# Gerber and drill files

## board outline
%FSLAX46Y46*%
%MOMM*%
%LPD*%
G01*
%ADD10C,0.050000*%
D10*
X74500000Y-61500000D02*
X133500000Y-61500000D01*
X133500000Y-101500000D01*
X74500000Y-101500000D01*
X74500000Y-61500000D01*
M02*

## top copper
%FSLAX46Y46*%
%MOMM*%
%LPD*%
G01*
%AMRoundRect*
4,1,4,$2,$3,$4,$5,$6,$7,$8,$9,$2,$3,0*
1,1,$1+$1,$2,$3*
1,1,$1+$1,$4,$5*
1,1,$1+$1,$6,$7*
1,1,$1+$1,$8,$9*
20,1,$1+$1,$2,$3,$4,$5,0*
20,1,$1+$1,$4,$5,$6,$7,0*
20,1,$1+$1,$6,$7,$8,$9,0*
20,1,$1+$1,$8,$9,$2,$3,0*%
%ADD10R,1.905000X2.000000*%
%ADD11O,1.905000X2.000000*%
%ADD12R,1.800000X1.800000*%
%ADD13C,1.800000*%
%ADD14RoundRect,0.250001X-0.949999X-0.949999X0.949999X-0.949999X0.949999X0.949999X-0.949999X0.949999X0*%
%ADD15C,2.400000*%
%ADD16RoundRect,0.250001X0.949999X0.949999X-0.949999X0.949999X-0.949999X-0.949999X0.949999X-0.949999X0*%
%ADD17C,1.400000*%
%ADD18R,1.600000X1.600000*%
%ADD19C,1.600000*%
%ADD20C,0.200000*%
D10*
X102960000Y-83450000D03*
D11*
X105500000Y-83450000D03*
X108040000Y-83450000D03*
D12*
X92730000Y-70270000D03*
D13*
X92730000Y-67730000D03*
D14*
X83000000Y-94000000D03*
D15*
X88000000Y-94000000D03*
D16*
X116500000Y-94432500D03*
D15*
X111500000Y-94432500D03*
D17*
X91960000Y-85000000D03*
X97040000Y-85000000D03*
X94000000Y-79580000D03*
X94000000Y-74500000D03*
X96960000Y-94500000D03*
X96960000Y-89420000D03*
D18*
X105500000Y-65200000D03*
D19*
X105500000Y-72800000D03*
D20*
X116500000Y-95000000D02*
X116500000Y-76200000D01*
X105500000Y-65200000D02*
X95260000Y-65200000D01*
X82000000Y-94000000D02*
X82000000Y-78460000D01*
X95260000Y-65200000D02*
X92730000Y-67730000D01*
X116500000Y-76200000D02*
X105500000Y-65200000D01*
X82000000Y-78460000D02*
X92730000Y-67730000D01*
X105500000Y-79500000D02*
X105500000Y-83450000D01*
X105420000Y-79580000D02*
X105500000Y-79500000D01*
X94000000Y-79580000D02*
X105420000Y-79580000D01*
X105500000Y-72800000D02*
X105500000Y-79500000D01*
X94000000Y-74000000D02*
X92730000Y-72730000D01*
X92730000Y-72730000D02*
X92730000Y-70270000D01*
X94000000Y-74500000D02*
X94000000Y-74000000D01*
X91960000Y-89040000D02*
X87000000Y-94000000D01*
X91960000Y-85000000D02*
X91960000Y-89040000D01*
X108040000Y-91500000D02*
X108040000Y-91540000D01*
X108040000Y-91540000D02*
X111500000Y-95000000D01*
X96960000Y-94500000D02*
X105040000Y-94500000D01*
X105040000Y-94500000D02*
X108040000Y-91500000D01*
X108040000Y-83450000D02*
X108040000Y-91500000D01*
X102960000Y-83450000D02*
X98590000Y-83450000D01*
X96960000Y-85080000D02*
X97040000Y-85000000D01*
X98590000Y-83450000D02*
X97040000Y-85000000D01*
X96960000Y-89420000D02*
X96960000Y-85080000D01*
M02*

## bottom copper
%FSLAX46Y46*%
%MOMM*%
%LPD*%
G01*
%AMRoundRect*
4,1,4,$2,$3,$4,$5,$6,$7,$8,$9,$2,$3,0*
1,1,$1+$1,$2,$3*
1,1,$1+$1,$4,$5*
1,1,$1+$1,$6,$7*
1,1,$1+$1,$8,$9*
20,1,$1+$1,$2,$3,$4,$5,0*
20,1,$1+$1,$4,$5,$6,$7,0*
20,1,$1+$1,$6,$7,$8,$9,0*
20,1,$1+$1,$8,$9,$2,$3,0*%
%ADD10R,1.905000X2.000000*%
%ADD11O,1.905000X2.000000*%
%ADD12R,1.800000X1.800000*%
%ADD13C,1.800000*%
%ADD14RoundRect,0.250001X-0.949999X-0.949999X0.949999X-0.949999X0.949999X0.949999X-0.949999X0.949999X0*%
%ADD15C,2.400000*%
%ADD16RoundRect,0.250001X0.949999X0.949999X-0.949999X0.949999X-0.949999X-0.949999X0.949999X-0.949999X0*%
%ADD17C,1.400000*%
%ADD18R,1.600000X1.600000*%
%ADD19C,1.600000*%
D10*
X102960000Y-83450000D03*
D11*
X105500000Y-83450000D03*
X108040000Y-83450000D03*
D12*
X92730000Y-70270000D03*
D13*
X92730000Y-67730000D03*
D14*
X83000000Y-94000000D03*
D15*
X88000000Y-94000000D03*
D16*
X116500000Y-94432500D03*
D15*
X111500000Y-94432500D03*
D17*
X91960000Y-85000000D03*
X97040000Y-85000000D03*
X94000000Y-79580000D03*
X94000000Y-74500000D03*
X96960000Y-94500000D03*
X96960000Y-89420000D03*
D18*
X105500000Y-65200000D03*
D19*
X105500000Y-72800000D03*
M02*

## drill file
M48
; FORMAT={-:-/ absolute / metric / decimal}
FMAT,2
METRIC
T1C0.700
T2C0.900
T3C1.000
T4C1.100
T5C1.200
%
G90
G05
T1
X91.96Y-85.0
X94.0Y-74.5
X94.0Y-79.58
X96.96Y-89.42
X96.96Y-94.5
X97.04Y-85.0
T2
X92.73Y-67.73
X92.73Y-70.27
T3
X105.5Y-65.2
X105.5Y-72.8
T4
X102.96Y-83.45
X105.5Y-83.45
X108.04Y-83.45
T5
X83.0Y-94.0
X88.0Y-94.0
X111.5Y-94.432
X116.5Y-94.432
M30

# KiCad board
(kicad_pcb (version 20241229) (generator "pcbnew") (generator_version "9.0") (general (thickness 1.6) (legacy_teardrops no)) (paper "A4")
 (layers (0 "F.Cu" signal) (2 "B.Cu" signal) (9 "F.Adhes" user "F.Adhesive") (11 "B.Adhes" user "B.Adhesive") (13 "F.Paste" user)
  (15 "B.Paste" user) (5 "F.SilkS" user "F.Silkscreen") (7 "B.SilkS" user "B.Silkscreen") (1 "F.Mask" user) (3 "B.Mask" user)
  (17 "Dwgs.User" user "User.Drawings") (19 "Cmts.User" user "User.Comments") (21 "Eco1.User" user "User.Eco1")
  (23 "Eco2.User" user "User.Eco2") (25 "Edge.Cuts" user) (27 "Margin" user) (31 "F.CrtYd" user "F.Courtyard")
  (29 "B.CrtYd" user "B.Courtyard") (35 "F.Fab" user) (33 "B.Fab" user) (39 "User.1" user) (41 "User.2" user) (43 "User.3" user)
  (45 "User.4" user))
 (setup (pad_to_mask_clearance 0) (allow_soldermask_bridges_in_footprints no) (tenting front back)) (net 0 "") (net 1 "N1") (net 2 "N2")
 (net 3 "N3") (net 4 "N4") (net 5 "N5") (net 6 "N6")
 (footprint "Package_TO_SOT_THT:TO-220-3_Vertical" (layer "F.Cu") (at 102.96 83.45)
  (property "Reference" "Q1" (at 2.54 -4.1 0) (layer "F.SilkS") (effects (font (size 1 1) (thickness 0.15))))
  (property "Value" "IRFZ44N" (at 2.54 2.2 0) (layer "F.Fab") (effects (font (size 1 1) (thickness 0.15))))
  (pad "1" thru_hole rect (at 0 0) (size 1.905 2) (drill 1.1) (layers "*.Cu" "*.Mask") (remove_unused_layers no) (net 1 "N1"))
  (pad "2" thru_hole oval (at 2.54 0) (size 1.905 2) (drill 1.1) (layers "*.Cu" "*.Mask") (remove_unused_layers no) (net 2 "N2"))
  (pad "3" thru_hole oval (at 5.08 0) (size 1.905 2) (drill 1.1) (layers "*.Cu" "*.Mask") (remove_unused_layers no) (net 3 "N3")))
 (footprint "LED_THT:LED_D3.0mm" (layer "F.Cu") (at 92.73 70.27 90)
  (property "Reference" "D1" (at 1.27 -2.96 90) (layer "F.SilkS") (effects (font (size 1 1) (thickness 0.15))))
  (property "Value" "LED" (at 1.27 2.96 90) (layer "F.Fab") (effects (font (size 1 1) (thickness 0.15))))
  (pad "1" thru_hole rect (at 0 0 90) (size 1.8 1.8) (drill 0.9) (layers "*.Cu" "*.Mask") (remove_unused_layers no) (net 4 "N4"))
  (pad "2" thru_hole circle (at 2.54 0 90) (size 1.8 1.8) (drill 0.9) (layers "*.Cu" "*.Mask") (remove_unused_layers no) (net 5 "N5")))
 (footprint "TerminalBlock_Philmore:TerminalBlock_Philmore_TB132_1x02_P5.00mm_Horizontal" (layer "F.Cu") (at 83 94)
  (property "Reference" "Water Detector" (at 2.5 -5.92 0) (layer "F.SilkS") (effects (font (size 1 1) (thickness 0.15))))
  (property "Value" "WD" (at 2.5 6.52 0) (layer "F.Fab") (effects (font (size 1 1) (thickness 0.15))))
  (pad "1" thru_hole roundrect (at 0 0) (size 2.4 2.4) (drill 1.2) (layers "*.Cu" "*.Mask") (remove_unused_layers no)
   (roundrect_rratio 0.104167) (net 5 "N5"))
  (pad "2" thru_hole circle (at 5 0) (size 2.4 2.4) (drill 1.2) (layers "*.Cu" "*.Mask") (remove_unused_layers no) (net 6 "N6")))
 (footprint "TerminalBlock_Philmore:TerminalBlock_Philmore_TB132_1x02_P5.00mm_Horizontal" (layer "F.Cu") (at 116.5 94.4325 180)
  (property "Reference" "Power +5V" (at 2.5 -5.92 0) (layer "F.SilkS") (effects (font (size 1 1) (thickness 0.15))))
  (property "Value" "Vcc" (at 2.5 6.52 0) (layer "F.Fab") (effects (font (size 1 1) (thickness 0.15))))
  (pad "1" thru_hole roundrect (at 0 0 180) (size 2.4 2.4) (drill 1.2) (layers "*.Cu" "*.Mask") (remove_unused_layers no)
   (roundrect_rratio 0.104167) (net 5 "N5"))
  (pad "2" thru_hole circle (at 5 0 180) (size 2.4 2.4) (drill 1.2) (layers "*.Cu" "*.Mask") (remove_unused_layers no) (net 3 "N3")))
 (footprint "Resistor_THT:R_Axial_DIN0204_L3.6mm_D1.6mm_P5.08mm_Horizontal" (layer "F.Cu") (at 91.96 85)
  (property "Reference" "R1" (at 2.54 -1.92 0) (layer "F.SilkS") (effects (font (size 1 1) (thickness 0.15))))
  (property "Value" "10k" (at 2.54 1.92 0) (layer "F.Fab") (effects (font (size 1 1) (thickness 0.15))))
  (pad "1" thru_hole circle (at 0 0) (size 1.4 1.4) (drill 0.7) (layers "*.Cu" "*.Mask") (remove_unused_layers no) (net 6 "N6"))
  (pad "2" thru_hole circle (at 5.08 0) (size 1.4 1.4) (drill 0.7) (layers "*.Cu" "*.Mask") (remove_unused_layers no) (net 1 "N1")))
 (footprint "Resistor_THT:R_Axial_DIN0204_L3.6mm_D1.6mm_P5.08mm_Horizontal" (layer "F.Cu") (at 94 79.58 90)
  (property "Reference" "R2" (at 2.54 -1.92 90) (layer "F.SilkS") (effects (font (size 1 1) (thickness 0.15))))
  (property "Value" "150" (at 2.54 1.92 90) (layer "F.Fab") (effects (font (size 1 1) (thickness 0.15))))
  (pad "1" thru_hole circle (at 0 0 90) (size 1.4 1.4) (drill 0.7) (layers "*.Cu" "*.Mask") (remove_unused_layers no) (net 2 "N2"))
  (pad "2" thru_hole circle (at 5.08 0 90) (size 1.4 1.4) (drill 0.7) (layers "*.Cu" "*.Mask") (remove_unused_layers no) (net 4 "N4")))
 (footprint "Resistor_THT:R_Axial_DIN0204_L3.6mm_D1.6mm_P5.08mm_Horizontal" (layer "F.Cu") (at 96.96 94.5 90)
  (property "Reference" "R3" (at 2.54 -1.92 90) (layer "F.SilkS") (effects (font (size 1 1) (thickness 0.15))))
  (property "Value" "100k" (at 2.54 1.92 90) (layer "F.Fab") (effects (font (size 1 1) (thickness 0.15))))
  (pad "1" thru_hole circle (at 0 0 90) (size 1.4 1.4) (drill 0.7) (layers "*.Cu" "*.Mask") (remove_unused_layers no) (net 3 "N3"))
  (pad "2" thru_hole circle (at 5.08 0 90) (size 1.4 1.4) (drill 0.7) (layers "*.Cu" "*.Mask") (remove_unused_layers no) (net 1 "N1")))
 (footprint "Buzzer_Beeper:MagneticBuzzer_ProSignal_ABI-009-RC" (layer "F.Cu") (at 105.5 65.2 -90)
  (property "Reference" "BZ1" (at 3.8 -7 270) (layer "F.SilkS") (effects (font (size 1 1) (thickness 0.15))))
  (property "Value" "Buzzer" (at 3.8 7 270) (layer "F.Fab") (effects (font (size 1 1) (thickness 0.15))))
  (pad "1" thru_hole rect (at 0 0 270) (size 1.6 1.6) (drill 1) (layers "*.Cu" "*.Mask") (remove_unused_layers no) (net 5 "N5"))
  (pad "2" thru_hole circle (at 7.6 0 270) (size 1.6 1.6) (drill 1) (layers "*.Cu" "*.Mask") (remove_unused_layers no) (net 2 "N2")))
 (gr_rect (start 74.5 61.5) (end 133.5 101.5) (stroke (width 0.05) (type default)) (fill no) (layer "Edge.Cuts"))
 (segment (start 116.5 95) (end 116.5 76.2) (width 0.2) (layer "F.Cu") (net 5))
 (segment (start 105.5 65.2) (end 95.26 65.2) (width 0.2) (layer "F.Cu") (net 5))
 (segment (start 82 94) (end 82 78.46) (width 0.2) (layer "F.Cu") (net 5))
 (segment (start 95.26 65.2) (end 92.73 67.73) (width 0.2) (layer "F.Cu") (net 5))
 (segment (start 116.5 76.2) (end 105.5 65.2) (width 0.2) (layer "F.Cu") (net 5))
 (segment (start 82 78.46) (end 92.73 67.73) (width 0.2) (layer "F.Cu") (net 5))
 (segment (start 105.5 79.5) (end 105.5 83.45) (width 0.2) (layer "F.Cu") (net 2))
 (segment (start 105.42 79.58) (end 105.5 79.5) (width 0.2) (layer "F.Cu") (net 2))
 (segment (start 94 79.58) (end 105.42 79.58) (width 0.2) (layer "F.Cu") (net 2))
 (segment (start 105.5 72.8) (end 105.5 79.5) (width 0.2) (layer "F.Cu") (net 2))
 (segment (start 94 74) (end 92.73 72.73) (width 0.2) (layer "F.Cu") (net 4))
 (segment (start 92.73 72.73) (end 92.73 70.27) (width 0.2) (layer "F.Cu") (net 4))
 (segment (start 94 74.5) (end 94 74) (width 0.2) (layer "F.Cu") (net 4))
 (segment (start 91.96 89.04) (end 87 94) (width 0.2) (layer "F.Cu") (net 6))
 (segment (start 91.96 85) (end 91.96 89.04) (width 0.2) (layer "F.Cu") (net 6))
 (segment (start 108.04 91.5) (end 108.04 91.54) (width 0.2) (layer "F.Cu") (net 3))
 (segment (start 108.04 91.54) (end 111.5 95) (width 0.2) (layer "F.Cu") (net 3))
 (segment (start 96.96 94.5) (end 105.04 94.5) (width 0.2) (layer "F.Cu") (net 3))
 (segment (start 105.04 94.5) (end 108.04 91.5) (width 0.2) (layer "F.Cu") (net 3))
 (segment (start 108.04 83.45) (end 108.04 91.5) (width 0.2) (layer "F.Cu") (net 3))
 (segment (start 102.96 83.45) (end 98.59 83.45) (width 0.2) (layer "F.Cu") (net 1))
 (segment (start 96.96 85.08) (end 97.04 85) (width 0.2) (layer "F.Cu") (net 1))
 (segment (start 98.59 83.45) (end 97.04 85) (width 0.2) (layer "F.Cu") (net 1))
 (segment (start 96.96 89.42) (end 96.96 85.08) (width 0.2) (layer "F.Cu") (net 1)))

